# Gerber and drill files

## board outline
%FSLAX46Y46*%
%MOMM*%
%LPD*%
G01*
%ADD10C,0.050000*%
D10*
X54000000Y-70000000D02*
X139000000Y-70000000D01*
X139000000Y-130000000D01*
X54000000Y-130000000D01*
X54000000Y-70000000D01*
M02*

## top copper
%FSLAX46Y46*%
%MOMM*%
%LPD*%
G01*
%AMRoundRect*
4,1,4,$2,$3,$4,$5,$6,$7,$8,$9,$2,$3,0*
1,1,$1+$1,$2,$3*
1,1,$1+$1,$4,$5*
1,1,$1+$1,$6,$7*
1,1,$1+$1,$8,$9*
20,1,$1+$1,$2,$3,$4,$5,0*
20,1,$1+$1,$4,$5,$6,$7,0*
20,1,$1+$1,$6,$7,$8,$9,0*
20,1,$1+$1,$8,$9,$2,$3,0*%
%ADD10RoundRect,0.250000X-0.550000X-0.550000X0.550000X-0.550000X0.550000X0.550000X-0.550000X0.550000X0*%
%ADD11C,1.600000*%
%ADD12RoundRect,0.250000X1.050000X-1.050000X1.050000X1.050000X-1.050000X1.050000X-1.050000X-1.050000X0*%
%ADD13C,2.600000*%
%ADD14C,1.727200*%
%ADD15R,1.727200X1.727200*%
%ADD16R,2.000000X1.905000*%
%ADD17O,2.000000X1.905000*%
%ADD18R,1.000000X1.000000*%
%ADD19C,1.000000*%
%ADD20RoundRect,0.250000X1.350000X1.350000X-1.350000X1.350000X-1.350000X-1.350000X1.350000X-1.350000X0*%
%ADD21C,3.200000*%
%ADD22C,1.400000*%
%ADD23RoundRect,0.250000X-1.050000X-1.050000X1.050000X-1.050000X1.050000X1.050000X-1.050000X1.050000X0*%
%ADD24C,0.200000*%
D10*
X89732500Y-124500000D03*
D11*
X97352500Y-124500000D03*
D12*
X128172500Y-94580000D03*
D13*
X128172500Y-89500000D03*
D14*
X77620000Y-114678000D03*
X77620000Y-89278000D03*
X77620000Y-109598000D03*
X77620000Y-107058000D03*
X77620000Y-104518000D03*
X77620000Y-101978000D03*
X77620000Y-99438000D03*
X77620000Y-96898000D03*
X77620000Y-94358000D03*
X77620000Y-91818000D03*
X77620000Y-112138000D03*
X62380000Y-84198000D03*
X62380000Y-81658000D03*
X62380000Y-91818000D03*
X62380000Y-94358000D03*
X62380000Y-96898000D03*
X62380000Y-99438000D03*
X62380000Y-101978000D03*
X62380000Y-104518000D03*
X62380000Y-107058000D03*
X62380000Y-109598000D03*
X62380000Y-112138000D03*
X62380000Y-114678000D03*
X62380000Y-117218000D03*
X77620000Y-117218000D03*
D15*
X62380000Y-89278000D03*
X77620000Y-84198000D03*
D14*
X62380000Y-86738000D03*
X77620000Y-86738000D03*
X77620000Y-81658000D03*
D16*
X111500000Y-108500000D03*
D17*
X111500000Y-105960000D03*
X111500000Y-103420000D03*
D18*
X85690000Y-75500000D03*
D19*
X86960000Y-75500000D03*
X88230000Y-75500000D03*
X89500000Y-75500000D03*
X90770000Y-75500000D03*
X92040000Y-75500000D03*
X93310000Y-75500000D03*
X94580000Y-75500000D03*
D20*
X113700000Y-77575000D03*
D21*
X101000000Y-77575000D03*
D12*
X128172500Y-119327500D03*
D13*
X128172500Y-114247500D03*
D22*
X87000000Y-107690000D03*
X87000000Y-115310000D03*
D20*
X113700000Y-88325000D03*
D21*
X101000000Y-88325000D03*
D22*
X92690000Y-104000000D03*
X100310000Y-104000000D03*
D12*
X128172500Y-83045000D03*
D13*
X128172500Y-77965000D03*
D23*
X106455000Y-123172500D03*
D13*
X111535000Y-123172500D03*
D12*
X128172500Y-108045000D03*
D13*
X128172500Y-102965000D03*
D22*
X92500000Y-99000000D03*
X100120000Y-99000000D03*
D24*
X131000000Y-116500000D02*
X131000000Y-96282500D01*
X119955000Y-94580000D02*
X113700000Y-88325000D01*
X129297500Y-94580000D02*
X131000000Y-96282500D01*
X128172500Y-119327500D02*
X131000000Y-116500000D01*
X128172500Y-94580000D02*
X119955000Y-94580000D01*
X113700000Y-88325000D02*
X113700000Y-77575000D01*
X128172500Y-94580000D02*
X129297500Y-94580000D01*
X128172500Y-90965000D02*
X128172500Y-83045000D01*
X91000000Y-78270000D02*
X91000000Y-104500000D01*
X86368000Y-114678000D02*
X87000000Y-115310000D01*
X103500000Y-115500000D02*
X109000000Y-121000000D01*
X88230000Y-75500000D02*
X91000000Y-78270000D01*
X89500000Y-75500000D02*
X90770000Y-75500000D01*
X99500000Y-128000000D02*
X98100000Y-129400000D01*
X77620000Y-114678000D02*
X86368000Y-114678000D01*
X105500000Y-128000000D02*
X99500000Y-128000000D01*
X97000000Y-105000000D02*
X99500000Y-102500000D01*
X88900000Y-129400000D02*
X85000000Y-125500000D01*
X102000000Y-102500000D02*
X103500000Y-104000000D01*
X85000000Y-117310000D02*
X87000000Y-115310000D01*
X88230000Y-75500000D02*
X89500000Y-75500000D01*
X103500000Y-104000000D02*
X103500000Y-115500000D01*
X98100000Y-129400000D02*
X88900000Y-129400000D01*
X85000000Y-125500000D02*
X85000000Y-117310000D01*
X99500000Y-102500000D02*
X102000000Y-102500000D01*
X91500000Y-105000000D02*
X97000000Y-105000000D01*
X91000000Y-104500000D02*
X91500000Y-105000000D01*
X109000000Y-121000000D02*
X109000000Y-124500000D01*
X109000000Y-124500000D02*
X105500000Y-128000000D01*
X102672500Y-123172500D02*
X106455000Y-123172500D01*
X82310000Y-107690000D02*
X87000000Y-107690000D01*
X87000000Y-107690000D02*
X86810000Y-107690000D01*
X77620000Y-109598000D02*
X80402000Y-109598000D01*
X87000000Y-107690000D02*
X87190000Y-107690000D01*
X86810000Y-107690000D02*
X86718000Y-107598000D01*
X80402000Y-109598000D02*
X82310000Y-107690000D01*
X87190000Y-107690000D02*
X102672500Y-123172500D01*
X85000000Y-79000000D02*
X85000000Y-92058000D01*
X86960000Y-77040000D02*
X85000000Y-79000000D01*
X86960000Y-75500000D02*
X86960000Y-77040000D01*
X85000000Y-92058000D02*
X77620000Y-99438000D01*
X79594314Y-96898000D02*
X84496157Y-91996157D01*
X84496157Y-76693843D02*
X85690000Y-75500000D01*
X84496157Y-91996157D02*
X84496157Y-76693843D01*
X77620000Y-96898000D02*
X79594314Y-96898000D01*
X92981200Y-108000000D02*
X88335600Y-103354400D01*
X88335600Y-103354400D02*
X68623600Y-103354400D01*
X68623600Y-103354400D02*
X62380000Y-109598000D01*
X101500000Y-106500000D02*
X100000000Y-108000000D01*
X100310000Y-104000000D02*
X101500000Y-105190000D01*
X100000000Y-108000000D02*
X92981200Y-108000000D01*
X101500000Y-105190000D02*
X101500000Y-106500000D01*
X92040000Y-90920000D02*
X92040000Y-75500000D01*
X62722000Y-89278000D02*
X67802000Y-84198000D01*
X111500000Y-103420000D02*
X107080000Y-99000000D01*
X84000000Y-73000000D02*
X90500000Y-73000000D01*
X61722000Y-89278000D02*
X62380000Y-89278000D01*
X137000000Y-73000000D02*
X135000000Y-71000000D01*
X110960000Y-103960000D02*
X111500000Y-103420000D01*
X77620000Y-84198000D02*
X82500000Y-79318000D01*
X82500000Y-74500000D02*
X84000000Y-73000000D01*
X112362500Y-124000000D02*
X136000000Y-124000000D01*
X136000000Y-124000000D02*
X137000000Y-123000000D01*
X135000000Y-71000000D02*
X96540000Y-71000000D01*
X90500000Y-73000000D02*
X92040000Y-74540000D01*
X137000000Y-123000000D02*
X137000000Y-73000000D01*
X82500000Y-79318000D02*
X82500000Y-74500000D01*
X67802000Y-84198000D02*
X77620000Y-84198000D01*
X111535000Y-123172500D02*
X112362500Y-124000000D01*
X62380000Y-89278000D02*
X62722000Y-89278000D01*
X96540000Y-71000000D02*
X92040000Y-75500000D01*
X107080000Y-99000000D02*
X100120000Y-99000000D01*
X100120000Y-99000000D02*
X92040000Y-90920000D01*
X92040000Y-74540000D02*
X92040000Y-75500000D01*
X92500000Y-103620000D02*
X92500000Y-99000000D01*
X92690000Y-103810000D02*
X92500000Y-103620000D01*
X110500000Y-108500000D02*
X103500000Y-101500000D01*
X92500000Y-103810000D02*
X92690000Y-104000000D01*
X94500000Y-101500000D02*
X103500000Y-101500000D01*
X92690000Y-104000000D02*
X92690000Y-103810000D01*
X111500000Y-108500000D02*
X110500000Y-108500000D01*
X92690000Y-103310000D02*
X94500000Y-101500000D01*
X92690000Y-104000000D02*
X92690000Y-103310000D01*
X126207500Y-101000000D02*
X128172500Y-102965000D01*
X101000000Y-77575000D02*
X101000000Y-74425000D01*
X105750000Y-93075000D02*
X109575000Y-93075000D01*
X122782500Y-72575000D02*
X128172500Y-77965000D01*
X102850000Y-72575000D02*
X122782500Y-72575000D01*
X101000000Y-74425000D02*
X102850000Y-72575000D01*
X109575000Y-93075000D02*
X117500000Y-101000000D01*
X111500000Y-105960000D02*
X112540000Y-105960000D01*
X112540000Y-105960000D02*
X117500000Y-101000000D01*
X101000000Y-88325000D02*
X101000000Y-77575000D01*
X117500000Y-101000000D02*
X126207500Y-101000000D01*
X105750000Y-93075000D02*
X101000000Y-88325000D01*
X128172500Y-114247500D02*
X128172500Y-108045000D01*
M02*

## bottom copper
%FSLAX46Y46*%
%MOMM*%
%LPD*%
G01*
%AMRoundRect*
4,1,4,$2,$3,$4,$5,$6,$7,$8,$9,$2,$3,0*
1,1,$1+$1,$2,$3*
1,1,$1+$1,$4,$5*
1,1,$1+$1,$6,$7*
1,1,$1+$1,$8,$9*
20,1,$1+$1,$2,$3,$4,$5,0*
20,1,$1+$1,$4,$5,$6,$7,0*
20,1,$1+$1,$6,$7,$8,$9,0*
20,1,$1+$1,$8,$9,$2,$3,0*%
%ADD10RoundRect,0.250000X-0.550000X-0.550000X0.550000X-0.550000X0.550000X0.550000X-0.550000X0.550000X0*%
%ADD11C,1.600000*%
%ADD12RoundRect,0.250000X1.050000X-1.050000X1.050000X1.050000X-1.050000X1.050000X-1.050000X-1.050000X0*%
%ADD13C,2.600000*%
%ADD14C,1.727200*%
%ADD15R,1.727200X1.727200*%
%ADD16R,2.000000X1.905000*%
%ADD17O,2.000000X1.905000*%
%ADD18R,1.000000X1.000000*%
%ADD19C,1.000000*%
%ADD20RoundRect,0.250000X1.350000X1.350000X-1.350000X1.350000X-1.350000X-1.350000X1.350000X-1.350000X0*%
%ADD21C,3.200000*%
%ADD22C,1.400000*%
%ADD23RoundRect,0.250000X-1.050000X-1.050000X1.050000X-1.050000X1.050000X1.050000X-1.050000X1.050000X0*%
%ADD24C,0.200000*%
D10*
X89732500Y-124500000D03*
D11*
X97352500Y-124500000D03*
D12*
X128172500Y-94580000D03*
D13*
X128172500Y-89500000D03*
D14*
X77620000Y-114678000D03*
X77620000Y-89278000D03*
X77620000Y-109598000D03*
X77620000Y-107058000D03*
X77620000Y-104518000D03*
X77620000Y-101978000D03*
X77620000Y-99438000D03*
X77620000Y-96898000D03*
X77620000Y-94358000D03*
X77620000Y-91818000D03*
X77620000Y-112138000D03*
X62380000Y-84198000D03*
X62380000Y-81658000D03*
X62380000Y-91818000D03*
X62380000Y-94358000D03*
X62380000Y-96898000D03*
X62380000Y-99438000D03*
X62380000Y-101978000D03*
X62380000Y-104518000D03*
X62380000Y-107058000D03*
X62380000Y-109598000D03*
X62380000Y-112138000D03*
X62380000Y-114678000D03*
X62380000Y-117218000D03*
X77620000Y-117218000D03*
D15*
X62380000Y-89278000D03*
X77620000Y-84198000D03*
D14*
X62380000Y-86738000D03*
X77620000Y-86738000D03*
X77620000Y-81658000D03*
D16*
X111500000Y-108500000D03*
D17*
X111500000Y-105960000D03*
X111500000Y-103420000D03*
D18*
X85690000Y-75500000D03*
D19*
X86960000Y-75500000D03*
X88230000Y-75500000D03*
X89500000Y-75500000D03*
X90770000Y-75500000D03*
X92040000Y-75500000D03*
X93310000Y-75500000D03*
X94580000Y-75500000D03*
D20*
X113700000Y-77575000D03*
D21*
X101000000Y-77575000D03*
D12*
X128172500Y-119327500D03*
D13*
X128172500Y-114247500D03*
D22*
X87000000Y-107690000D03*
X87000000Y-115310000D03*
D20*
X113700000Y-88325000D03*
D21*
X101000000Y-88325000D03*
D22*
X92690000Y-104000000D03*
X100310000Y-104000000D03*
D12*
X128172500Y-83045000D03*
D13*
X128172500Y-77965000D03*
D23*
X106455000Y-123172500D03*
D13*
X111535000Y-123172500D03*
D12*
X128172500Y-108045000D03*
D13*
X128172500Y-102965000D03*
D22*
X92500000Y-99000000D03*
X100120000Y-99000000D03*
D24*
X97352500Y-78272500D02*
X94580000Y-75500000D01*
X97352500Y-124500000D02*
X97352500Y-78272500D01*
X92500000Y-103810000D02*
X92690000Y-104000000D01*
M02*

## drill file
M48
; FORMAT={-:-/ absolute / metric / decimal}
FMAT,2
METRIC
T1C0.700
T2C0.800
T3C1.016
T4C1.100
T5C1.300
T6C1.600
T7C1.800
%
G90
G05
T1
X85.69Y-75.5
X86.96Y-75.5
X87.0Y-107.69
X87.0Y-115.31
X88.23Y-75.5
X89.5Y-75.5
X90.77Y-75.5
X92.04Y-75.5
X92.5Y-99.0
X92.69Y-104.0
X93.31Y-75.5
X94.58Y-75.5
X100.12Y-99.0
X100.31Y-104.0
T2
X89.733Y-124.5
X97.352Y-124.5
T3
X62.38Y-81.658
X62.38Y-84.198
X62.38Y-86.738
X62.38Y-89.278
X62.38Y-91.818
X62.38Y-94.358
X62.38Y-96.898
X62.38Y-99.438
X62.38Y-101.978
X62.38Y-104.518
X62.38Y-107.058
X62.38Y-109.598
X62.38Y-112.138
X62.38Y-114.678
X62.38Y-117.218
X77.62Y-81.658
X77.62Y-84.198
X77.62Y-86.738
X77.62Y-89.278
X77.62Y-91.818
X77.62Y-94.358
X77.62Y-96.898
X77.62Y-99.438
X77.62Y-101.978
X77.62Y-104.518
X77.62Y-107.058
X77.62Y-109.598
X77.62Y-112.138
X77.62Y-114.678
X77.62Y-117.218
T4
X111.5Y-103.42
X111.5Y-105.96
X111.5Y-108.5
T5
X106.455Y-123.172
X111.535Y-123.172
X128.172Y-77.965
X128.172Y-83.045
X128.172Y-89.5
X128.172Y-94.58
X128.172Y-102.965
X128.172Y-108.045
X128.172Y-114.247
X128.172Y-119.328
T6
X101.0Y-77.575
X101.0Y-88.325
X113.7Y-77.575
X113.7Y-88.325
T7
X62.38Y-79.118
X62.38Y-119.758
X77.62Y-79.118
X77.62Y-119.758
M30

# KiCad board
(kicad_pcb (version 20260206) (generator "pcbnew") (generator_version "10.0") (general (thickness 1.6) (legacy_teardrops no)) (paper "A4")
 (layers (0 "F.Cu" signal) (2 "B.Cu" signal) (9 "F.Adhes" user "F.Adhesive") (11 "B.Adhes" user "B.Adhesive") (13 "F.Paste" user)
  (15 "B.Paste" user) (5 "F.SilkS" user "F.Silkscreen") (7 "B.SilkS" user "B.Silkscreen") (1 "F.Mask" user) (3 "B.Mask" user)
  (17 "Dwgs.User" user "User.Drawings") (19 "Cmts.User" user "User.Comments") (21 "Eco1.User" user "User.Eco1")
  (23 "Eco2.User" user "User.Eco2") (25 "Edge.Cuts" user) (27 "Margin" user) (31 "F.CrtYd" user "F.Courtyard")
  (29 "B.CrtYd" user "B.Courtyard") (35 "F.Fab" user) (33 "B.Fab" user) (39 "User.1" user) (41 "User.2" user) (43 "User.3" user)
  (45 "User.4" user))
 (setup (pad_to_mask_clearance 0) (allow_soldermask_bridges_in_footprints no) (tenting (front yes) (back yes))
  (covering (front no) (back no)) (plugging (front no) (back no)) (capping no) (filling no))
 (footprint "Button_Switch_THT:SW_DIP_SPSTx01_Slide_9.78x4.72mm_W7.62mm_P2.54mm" (layer "F.Cu") (at 89.7325 124.5)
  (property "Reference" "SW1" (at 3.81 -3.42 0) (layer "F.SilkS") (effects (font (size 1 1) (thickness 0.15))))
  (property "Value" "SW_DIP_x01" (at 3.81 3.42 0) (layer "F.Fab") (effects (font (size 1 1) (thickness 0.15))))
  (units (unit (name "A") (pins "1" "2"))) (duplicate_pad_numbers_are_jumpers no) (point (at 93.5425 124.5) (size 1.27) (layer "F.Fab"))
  (pad "1" thru_hole roundrect (at 0 0) (size 1.6 1.6) (drill 0.8) (layers "*.Cu" "*.Mask") (remove_unused_layers no)
   (roundrect_rratio 0.15625) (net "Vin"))
  (pad "2" thru_hole circle (at 7.62 0) (size 1.6 1.6) (drill 0.8) (layers "*.Cu" "*.Mask") (remove_unused_layers no) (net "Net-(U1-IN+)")))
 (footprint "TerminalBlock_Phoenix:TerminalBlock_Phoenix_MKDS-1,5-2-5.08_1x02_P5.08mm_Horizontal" (layer "F.Cu") (at 128.1725 94.58 90)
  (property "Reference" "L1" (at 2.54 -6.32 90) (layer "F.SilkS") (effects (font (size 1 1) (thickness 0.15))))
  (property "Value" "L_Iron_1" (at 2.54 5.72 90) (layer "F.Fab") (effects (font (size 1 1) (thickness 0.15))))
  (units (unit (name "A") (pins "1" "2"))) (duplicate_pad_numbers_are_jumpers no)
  (pad "1" thru_hole roundrect (at 0 0 90) (size 2.6 2.6) (drill 1.3) (layers "*.Cu" "*.Mask") (remove_unused_layers no)
   (roundrect_rratio 0.096154) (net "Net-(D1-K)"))
  (pad "2" thru_hole circle (at 5.08 0 90) (size 2.6 2.6) (drill 1.3) (layers "*.Cu" "*.Mask") (remove_unused_layers no)
   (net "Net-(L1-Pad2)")))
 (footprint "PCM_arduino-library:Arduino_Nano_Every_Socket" (layer "F.Cu") (at 70 121.028)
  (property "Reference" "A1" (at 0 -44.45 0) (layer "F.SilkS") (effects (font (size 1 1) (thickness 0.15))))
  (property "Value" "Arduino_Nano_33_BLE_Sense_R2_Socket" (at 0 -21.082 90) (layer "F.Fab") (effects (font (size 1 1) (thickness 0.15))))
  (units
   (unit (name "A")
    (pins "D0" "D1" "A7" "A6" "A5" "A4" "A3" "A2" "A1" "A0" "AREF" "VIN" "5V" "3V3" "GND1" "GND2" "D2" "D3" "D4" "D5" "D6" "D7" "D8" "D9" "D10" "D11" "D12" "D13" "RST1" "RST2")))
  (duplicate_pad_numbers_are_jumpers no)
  (pad "" np_thru_hole circle (at -7.62 -41.91) (size 1.8 1.8) (drill 1.8) (layers "*.Cu" "*.Mask"))
  (pad "" np_thru_hole circle (at -7.62 -1.27) (size 1.8 1.8) (drill 1.8) (layers "*.Cu" "*.Mask"))
  (pad "" np_thru_hole circle (at 7.62 -41.91) (size 1.8 1.8) (drill 1.8) (layers "*.Cu" "*.Mask"))
  (pad "" np_thru_hole circle (at 7.62 -1.27) (size 1.8 1.8) (drill 1.8) (layers "*.Cu" "*.Mask"))
  (pad "3V3" thru_hole circle (at 7.62 -6.35) (size 1.7272 1.7272) (drill 1.016) (layers "*.Cu" "*.Mask") (remove_unused_layers no)
   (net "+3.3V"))
  (pad "5V" thru_hole circle (at 7.62 -31.75) (size 1.7272 1.7272) (drill 1.016) (layers "*.Cu" "*.Mask") (remove_unused_layers no)
   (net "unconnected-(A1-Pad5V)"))
  (pad "A0" thru_hole circle (at 7.62 -11.43) (size 1.7272 1.7272) (drill 1.016) (layers "*.Cu" "*.Mask") (remove_unused_layers no)
   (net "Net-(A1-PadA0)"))
  (pad "A1" thru_hole circle (at 7.62 -13.97) (size 1.7272 1.7272) (drill 1.016) (layers "*.Cu" "*.Mask") (remove_unused_layers no)
   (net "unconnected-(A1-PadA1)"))
  (pad "A2" thru_hole circle (at 7.62 -16.51) (size 1.7272 1.7272) (drill 1.016) (layers "*.Cu" "*.Mask") (remove_unused_layers no)
   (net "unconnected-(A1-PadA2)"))
  (pad "A3" thru_hole circle (at 7.62 -19.05) (size 1.7272 1.7272) (drill 1.016) (layers "*.Cu" "*.Mask") (remove_unused_layers no)
   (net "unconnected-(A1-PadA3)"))
  (pad "A4" thru_hole circle (at 7.62 -21.59) (size 1.7272 1.7272) (drill 1.016) (layers "*.Cu" "*.Mask") (remove_unused_layers no)
   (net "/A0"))
  (pad "A5" thru_hole circle (at 7.62 -24.13) (size 1.7272 1.7272) (drill 1.016) (layers "*.Cu" "*.Mask") (remove_unused_layers no)
   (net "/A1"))
  (pad "A6" thru_hole circle (at 7.62 -26.67) (size 1.7272 1.7272) (drill 1.016) (layers "*.Cu" "*.Mask") (remove_unused_layers no)
   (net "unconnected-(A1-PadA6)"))
  (pad "A7" thru_hole circle (at 7.62 -29.21) (size 1.7272 1.7272) (drill 1.016) (layers "*.Cu" "*.Mask") (remove_unused_layers no)
   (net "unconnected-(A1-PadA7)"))
  (pad "AREF" thru_hole circle (at 7.62 -8.89) (size 1.7272 1.7272) (drill 1.016) (layers "*.Cu" "*.Mask") (remove_unused_layers no)
   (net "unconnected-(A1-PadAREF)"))
  (pad "D0" thru_hole circle (at -7.62 -36.83) (size 1.7272 1.7272) (drill 1.016) (layers "*.Cu" "*.Mask") (remove_unused_layers no)
   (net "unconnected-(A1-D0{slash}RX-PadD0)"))
  (pad "D1" thru_hole circle (at -7.62 -39.37) (size 1.7272 1.7272) (drill 1.016) (layers "*.Cu" "*.Mask") (remove_unused_layers no)
   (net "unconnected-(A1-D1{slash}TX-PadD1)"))
  (pad "D2" thru_hole circle (at -7.62 -29.21) (size 1.7272 1.7272) (drill 1.016) (layers "*.Cu" "*.Mask") (remove_unused_layers no)
   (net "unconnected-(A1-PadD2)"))
  (pad "D3" thru_hole circle (at -7.62 -26.67) (size 1.7272 1.7272) (drill 1.016) (layers "*.Cu" "*.Mask") (remove_unused_layers no)
   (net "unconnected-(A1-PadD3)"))
  (pad "D4" thru_hole circle (at -7.62 -24.13) (size 1.7272 1.7272) (drill 1.016) (layers "*.Cu" "*.Mask") (remove_unused_layers no)
   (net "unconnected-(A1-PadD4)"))
  (pad "D5" thru_hole circle (at -7.62 -21.59) (size 1.7272 1.7272) (drill 1.016) (layers "*.Cu" "*.Mask") (remove_unused_layers no)
   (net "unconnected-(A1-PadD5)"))
  (pad "D6" thru_hole circle (at -7.62 -19.05) (size 1.7272 1.7272) (drill 1.016) (layers "*.Cu" "*.Mask") (remove_unused_layers no)
   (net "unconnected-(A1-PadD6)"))
  (pad "D7" thru_hole circle (at -7.62 -16.51) (size 1.7272 1.7272) (drill 1.016) (layers "*.Cu" "*.Mask") (remove_unused_layers no)
   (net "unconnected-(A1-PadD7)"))
  (pad "D8" thru_hole circle (at -7.62 -13.97) (size 1.7272 1.7272) (drill 1.016) (layers "*.Cu" "*.Mask") (remove_unused_layers no)
   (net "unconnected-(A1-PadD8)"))
  (pad "D9" thru_hole circle (at -7.62 -11.43) (size 1.7272 1.7272) (drill 1.016) (layers "*.Cu" "*.Mask") (remove_unused_layers no)
   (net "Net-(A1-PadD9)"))
  (pad "D10" thru_hole circle (at -7.62 -8.89) (size 1.7272 1.7272) (drill 1.016) (layers "*.Cu" "*.Mask") (remove_unused_layers no)
   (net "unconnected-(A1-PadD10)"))
  (pad "D11" thru_hole circle (at -7.62 -6.35) (size 1.7272 1.7272) (drill 1.016) (layers "*.Cu" "*.Mask") (remove_unused_layers no)
   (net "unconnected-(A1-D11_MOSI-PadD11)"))
  (pad "D12" thru_hole circle (at -7.62 -3.81) (size 1.7272 1.7272) (drill 1.016) (layers "*.Cu" "*.Mask") (remove_unused_layers no)
   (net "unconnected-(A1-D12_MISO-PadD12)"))
  (pad "D13" thru_hole circle (at 7.62 -3.81) (size 1.7272 1.7272) (drill 1.016) (layers "*.Cu" "*.Mask") (remove_unused_layers no)
   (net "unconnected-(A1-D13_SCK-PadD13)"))
  (pad "GND1" thru_hole rect (at -7.62 -31.75) (size 1.7272 1.7272) (drill 1.016) (layers "*.Cu" "*.Mask") (remove_unused_layers no)
   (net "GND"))
  (pad "GND2" thru_hole rect (at 7.62 -36.83) (size 1.7272 1.7272) (drill 1.016) (layers "*.Cu" "*.Mask") (remove_unused_layers no)
   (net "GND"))
  (pad "RST1" thru_hole circle (at -7.62 -34.29) (size 1.7272 1.7272) (drill 1.016) (layers "*.Cu" "*.Mask") (remove_unused_layers no)
   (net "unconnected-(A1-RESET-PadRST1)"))
  (pad "RST2" thru_hole circle (at 7.62 -34.29) (size 1.7272 1.7272) (drill 1.016) (layers "*.Cu" "*.Mask") (remove_unused_layers no)
   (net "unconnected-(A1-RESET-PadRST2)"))
  (pad "VIN" thru_hole circle (at 7.62 -39.37) (size 1.7272 1.7272) (drill 1.016) (layers "*.Cu" "*.Mask") (remove_unused_layers no)
   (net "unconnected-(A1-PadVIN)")))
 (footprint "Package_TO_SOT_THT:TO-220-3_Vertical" (layer "F.Cu") (at 111.5 108.5 90)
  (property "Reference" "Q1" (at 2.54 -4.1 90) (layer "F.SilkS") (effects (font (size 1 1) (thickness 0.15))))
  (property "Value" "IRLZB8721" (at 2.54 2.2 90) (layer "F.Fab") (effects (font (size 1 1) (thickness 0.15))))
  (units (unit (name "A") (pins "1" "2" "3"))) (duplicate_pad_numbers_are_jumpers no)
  (pad "1" thru_hole rect (at 0 0 90) (size 1.905 2) (drill 1.1) (layers "*.Cu" "*.Mask") (remove_unused_layers no) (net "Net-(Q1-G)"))
  (pad "2" thru_hole oval (at 2.54 0 90) (size 1.905 2) (drill 1.1) (layers "*.Cu" "*.Mask") (remove_unused_layers no) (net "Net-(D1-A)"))
  (pad "3" thru_hole oval (at 5.08 0 90) (size 1.905 2) (drill 1.1) (layers "*.Cu" "*.Mask") (remove_unused_layers no) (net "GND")))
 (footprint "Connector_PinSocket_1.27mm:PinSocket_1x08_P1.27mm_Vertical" (layer "F.Cu") (at 85.69 75.5 90)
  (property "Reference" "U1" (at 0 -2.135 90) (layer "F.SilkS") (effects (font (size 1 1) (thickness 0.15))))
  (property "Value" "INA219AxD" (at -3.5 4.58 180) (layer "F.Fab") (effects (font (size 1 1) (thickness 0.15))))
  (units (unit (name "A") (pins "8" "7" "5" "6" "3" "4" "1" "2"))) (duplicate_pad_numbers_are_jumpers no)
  (pad "1" thru_hole rect (at 0 0 90) (size 1 1) (drill 0.7) (layers "*.Cu" "*.Mask") (remove_unused_layers no) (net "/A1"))
  (pad "2" thru_hole circle (at 0 1.27 90) (size 1 1) (drill 0.7) (layers "*.Cu" "*.Mask") (remove_unused_layers no) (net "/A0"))
  (pad "3" thru_hole circle (at 0 2.54 90) (size 1 1) (drill 0.7) (layers "*.Cu" "*.Mask") (remove_unused_layers no) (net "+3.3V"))
  (pad "4" thru_hole circle (at 0 3.81 90) (size 1 1) (drill 0.7) (layers "*.Cu" "*.Mask") (remove_unused_layers no) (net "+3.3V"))
  (pad "5" thru_hole circle (at 0 5.08 90) (size 1 1) (drill 0.7) (layers "*.Cu" "*.Mask") (remove_unused_layers no) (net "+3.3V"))
  (pad "6" thru_hole circle (at 0 6.35 90) (size 1 1) (drill 0.7) (layers "*.Cu" "*.Mask") (remove_unused_layers no) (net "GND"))
  (pad "7" thru_hole circle (at 0 7.62 90) (size 1 1) (drill 0.7) (layers "*.Cu" "*.Mask") (remove_unused_layers no) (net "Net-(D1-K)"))
  (pad "8" thru_hole circle (at 0 8.89 90) (size 1 1) (drill 0.7) (layers "*.Cu" "*.Mask") (remove_unused_layers no) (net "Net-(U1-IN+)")))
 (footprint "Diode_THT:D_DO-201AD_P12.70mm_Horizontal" (layer "F.Cu") (at 113.7 77.575 180)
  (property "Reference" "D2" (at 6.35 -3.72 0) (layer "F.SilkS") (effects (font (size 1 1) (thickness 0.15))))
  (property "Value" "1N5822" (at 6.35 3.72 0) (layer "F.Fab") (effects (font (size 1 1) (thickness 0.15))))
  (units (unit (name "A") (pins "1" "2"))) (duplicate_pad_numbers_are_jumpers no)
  (pad "1" thru_hole roundrect (at 0 0 180) (size 3.2 3.2) (drill 1.6) (layers "*.Cu" "*.Mask") (remove_unused_layers no)
   (roundrect_rratio 0.078125) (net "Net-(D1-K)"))
  (pad "2" thru_hole circle (at 12.7 0 180) (size 3.2 3.2) (drill 1.6) (layers "*.Cu" "*.Mask") (remove_unused_layers no) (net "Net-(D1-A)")))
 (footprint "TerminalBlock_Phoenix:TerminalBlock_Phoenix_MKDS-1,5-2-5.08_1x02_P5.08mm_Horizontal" (layer "F.Cu") (at 128.1725 119.3275 90)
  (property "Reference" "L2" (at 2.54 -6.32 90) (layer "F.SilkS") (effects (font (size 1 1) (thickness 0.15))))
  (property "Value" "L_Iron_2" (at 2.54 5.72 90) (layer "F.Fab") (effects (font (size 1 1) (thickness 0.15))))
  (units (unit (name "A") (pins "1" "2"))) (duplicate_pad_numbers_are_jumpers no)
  (pad "1" thru_hole roundrect (at 0 0 90) (size 2.6 2.6) (drill 1.3) (layers "*.Cu" "*.Mask") (remove_unused_layers no)
   (roundrect_rratio 0.096154) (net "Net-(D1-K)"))
  (pad "2" thru_hole circle (at 5.08 0 90) (size 2.6 2.6) (drill 1.3) (layers "*.Cu" "*.Mask") (remove_unused_layers no)
   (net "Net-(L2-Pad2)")))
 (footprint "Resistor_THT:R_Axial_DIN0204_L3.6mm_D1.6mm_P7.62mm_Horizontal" (layer "F.Cu") (at 87 107.69 -90)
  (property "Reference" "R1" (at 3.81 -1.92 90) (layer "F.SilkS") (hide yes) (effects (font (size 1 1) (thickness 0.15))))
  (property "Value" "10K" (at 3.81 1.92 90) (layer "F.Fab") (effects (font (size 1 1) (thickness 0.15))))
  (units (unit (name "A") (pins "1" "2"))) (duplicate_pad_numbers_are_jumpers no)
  (pad "1" thru_hole circle (at 0 0 270) (size 1.4 1.4) (drill 0.7) (layers "*.Cu" "*.Mask") (remove_unused_layers no)
   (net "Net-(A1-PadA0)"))
  (pad "2" thru_hole circle (at 7.62 0 270) (size 1.4 1.4) (drill 0.7) (layers "*.Cu" "*.Mask") (remove_unused_layers no) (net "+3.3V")))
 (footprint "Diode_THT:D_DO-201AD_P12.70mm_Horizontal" (layer "F.Cu") (at 113.7 88.325 180)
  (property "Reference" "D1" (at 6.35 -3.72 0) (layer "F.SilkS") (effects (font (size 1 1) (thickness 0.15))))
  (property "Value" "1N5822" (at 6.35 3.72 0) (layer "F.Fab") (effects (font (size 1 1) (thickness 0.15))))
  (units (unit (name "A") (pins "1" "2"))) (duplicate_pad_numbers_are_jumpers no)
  (pad "1" thru_hole roundrect (at 0 0 180) (size 3.2 3.2) (drill 1.6) (layers "*.Cu" "*.Mask") (remove_unused_layers no)
   (roundrect_rratio 0.078125) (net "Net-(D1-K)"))
  (pad "2" thru_hole circle (at 12.7 0 180) (size 3.2 3.2) (drill 1.6) (layers "*.Cu" "*.Mask") (remove_unused_layers no) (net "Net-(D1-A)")))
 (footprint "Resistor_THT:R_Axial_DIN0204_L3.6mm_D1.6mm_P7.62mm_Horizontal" (layer "F.Cu") (at 92.69 104)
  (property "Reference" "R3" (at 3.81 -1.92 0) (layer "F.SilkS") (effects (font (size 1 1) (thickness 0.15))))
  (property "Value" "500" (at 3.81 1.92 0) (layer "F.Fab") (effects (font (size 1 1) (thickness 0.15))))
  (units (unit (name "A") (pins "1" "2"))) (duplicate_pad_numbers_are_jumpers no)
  (pad "1" thru_hole circle (at 0 0) (size 1.4 1.4) (drill 0.7) (layers "*.Cu" "*.Mask") (remove_unused_layers no) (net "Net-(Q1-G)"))
  (pad "2" thru_hole circle (at 7.62 0) (size 1.4 1.4) (drill 0.7) (layers "*.Cu" "*.Mask") (remove_unused_layers no) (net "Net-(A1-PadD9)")))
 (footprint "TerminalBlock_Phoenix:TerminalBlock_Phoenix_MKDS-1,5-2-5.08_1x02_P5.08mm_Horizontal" (layer "F.Cu") (at 128.1725 83.045 90)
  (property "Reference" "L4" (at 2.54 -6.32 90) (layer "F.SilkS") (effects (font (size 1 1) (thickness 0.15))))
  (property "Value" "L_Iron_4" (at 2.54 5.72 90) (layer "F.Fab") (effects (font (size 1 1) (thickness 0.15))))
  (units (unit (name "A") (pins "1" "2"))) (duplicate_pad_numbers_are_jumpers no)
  (pad "1" thru_hole roundrect (at 0 0 90) (size 2.6 2.6) (drill 1.3) (layers "*.Cu" "*.Mask") (remove_unused_layers no)
   (roundrect_rratio 0.096154) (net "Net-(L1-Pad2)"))
  (pad "2" thru_hole circle (at 5.08 0 90) (size 2.6 2.6) (drill 1.3) (layers "*.Cu" "*.Mask") (remove_unused_layers no) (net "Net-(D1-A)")))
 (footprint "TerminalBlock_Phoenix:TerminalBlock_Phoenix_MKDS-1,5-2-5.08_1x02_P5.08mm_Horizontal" (layer "F.Cu") (at 106.455 123.1725)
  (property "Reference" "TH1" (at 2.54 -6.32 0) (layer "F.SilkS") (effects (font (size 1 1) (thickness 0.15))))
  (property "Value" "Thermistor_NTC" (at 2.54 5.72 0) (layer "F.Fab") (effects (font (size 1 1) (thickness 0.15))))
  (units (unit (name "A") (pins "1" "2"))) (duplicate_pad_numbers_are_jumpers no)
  (pad "1" thru_hole roundrect (at 0 0) (size 2.6 2.6) (drill 1.3) (layers "*.Cu" "*.Mask") (remove_unused_layers no)
   (roundrect_rratio 0.096154) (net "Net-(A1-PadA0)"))
  (pad "2" thru_hole circle (at 5.08 0) (size 2.6 2.6) (drill 1.3) (layers "*.Cu" "*.Mask") (remove_unused_layers no) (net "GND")))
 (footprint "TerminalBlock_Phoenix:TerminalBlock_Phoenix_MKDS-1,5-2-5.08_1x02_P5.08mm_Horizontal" (layer "F.Cu") (at 128.1725 108.045 90)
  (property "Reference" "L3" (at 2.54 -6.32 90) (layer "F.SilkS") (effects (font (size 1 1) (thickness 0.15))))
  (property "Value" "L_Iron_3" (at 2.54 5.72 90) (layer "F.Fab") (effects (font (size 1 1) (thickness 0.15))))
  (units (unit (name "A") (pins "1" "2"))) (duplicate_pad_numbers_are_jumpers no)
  (pad "1" thru_hole roundrect (at 0 0 90) (size 2.6 2.6) (drill 1.3) (layers "*.Cu" "*.Mask") (remove_unused_layers no)
   (roundrect_rratio 0.096154) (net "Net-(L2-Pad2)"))
  (pad "2" thru_hole circle (at 5.08 0 90) (size 2.6 2.6) (drill 1.3) (layers "*.Cu" "*.Mask") (remove_unused_layers no) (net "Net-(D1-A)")))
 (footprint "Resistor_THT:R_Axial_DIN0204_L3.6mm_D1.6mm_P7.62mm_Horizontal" (layer "F.Cu") (at 92.5 99)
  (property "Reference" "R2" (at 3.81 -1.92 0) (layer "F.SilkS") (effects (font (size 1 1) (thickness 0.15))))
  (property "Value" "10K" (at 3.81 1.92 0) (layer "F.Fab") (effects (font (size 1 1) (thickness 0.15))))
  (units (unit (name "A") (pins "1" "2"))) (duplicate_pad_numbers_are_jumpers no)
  (pad "1" thru_hole circle (at 0 0) (size 1.4 1.4) (drill 0.7) (layers "*.Cu" "*.Mask") (remove_unused_layers no) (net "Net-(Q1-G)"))
  (pad "2" thru_hole circle (at 7.62 0) (size 1.4 1.4) (drill 0.7) (layers "*.Cu" "*.Mask") (remove_unused_layers no) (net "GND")))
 (gr_rect (start 54 70) (end 139 130) (stroke (width 0.05) (type default)) (fill no) (layer "Edge.Cuts"))
 (segment (start 97.3525 78.2725) (end 94.58 75.5) (width 0.2) (layer "B.Cu") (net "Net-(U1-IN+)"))
 (segment (start 97.3525 124.5) (end 97.3525 78.2725) (width 0.2) (layer "B.Cu") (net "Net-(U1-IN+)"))
 (segment (start 131 116.5) (end 131 96.2825) (width 0.2) (layer "F.Cu") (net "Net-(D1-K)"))
 (segment (start 119.955 94.58) (end 113.7 88.325) (width 0.2) (layer "F.Cu") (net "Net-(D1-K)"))
 (segment (start 129.2975 94.58) (end 131 96.2825) (width 0.2) (layer "F.Cu") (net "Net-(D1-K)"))
 (segment (start 128.1725 119.3275) (end 131 116.5) (width 0.2) (layer "F.Cu") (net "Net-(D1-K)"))
 (segment (start 128.1725 94.58) (end 119.955 94.58) (width 0.2) (layer "F.Cu") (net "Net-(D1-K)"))
 (segment (start 113.7 88.325) (end 113.7 77.575) (width 0.2) (layer "F.Cu") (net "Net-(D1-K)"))
 (segment (start 128.1725 94.58) (end 129.2975 94.58) (width 0.2) (layer "F.Cu") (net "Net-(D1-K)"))
 (segment (start 128.1725 90.965) (end 128.1725 83.045) (width 0.2) (layer "F.Cu") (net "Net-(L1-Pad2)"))
 (segment (start 91 78.27) (end 91 104.5) (width 0.2) (layer "F.Cu") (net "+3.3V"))
 (segment (start 86.368 114.678) (end 87 115.31) (width 0.2) (layer "F.Cu") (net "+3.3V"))
 (segment (start 103.5 115.5) (end 109 121) (width 0.2) (layer "F.Cu") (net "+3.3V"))
 (segment (start 88.23 75.5) (end 91 78.27) (width 0.2) (layer "F.Cu") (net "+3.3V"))
 (segment (start 89.5 75.5) (end 90.77 75.5) (width 0.2) (layer "F.Cu") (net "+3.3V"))
 (segment (start 99.5 128) (end 98.1 129.4) (width 0.2) (layer "F.Cu") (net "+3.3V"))
 (segment (start 77.62 114.678) (end 86.368 114.678) (width 0.2) (layer "F.Cu") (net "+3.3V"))
 (segment (start 105.5 128) (end 99.5 128) (width 0.2) (layer "F.Cu") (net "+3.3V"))
 (segment (start 97 105) (end 99.5 102.5) (width 0.2) (layer "F.Cu") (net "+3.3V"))
 (segment (start 88.9 129.4) (end 85 125.5) (width 0.2) (layer "F.Cu") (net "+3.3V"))
 (segment (start 102 102.5) (end 103.5 104) (width 0.2) (layer "F.Cu") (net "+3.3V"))
 (segment (start 85 117.31) (end 87 115.31) (width 0.2) (layer "F.Cu") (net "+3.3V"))
 (segment (start 88.23 75.5) (end 89.5 75.5) (width 0.2) (layer "F.Cu") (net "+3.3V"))
 (segment (start 103.5 104) (end 103.5 115.5) (width 0.2) (layer "F.Cu") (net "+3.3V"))
 (segment (start 98.1 129.4) (end 88.9 129.4) (width 0.2) (layer "F.Cu") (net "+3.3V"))
 (segment (start 85 125.5) (end 85 117.31) (width 0.2) (layer "F.Cu") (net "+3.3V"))
 (segment (start 99.5 102.5) (end 102 102.5) (width 0.2) (layer "F.Cu") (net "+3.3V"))
 (segment (start 91.5 105) (end 97 105) (width 0.2) (layer "F.Cu") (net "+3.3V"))
 (segment (start 91 104.5) (end 91.5 105) (width 0.2) (layer "F.Cu") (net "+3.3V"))
 (segment (start 109 121) (end 109 124.5) (width 0.2) (layer "F.Cu") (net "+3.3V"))
 (segment (start 109 124.5) (end 105.5 128) (width 0.2) (layer "F.Cu") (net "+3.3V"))
 (segment (start 102.6725 123.1725) (end 106.455 123.1725) (width 0.2) (layer "F.Cu") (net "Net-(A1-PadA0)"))
 (segment (start 82.31 107.69) (end 87 107.69) (width 0.2) (layer "F.Cu") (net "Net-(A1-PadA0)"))
 (segment (start 87 107.69) (end 86.81 107.69) (width 0.2) (layer "F.Cu") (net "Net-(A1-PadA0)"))
 (segment (start 77.62 109.598) (end 80.402 109.598) (width 0.2) (layer "F.Cu") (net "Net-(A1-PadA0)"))
 (segment (start 87 107.69) (end 87.19 107.69) (width 0.2) (layer "F.Cu") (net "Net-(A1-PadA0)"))
 (segment (start 86.81 107.69) (end 86.718 107.598) (width 0.2) (layer "F.Cu") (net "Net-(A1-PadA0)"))
 (segment (start 80.402 109.598) (end 82.31 107.69) (width 0.2) (layer "F.Cu") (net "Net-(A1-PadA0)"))
 (segment (start 87.19 107.69) (end 102.6725 123.1725) (width 0.2) (layer "F.Cu") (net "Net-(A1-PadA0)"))
 (segment (start 85 79) (end 85 92.058) (width 0.2) (layer "F.Cu") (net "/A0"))
 (segment (start 86.96 77.04) (end 85 79) (width 0.2) (layer "F.Cu") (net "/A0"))
 (segment (start 86.96 75.5) (end 86.96 77.04) (width 0.2) (layer "F.Cu") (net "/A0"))
 (segment (start 85 92.058) (end 77.62 99.438) (width 0.2) (layer "F.Cu") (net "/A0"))
 (segment (start 79.594314 96.898) (end 84.496157 91.996157) (width 0.2) (layer "F.Cu") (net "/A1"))
 (segment (start 84.496157 76.693843) (end 85.69 75.5) (width 0.2) (layer "F.Cu") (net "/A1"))
 (segment (start 84.496157 91.996157) (end 84.496157 76.693843) (width 0.2) (layer "F.Cu") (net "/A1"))
 (segment (start 77.62 96.898) (end 79.594314 96.898) (width 0.2) (layer "F.Cu") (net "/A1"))
 (segment (start 92.9812 108) (end 88.3356 103.3544) (width 0.2) (layer "F.Cu") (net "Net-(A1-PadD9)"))
 (segment (start 88.3356 103.3544) (end 68.6236 103.3544) (width 0.2) (layer "F.Cu") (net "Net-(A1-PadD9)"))
 (segment (start 68.6236 103.3544) (end 62.38 109.598) (width 0.2) (layer "F.Cu") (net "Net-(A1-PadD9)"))
 (segment (start 101.5 106.5) (end 100 108) (width 0.2) (layer "F.Cu") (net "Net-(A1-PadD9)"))
 (segment (start 100.31 104) (end 101.5 105.19) (width 0.2) (layer "F.Cu") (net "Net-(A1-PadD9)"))
 (segment (start 100 108) (end 92.9812 108) (width 0.2) (layer "F.Cu") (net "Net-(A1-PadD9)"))
 (segment (start 101.5 105.19) (end 101.5 106.5) (width 0.2) (layer "F.Cu") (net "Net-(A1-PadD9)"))
 (segment (start 92.04 90.92) (end 92.04 75.5) (width 0.2) (layer "F.Cu") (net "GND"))
 (segment (start 62.722 89.278) (end 67.802 84.198) (width 0.2) (layer "F.Cu") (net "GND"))
 (segment (start 111.5 103.42) (end 107.08 99) (width 0.2) (layer "F.Cu") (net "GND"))
 (segment (start 84 73) (end 90.5 73) (width 0.2) (layer "F.Cu") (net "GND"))
 (segment (start 61.722 89.278) (end 62.38 89.278) (width 0.2) (layer "F.Cu") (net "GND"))
 (segment (start 137 73) (end 135 71) (width 0.2) (layer "F.Cu") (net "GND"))
 (segment (start 110.96 103.96) (end 111.5 103.42) (width 0.2) (layer "F.Cu") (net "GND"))
 (segment (start 77.62 84.198) (end 82.5 79.318) (width 0.2) (layer "F.Cu") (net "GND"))
 (segment (start 82.5 74.5) (end 84 73) (width 0.2) (layer "F.Cu") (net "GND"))
 (segment (start 112.3625 124) (end 136 124) (width 0.2) (layer "F.Cu") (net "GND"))
 (segment (start 136 124) (end 137 123) (width 0.2) (layer "F.Cu") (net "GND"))
 (segment (start 135 71) (end 96.54 71) (width 0.2) (layer "F.Cu") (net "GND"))
 (segment (start 90.5 73) (end 92.04 74.54) (width 0.2) (layer "F.Cu") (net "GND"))
 (segment (start 137 123) (end 137 73) (width 0.2) (layer "F.Cu") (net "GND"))
 (segment (start 82.5 79.318) (end 82.5 74.5) (width 0.2) (layer "F.Cu") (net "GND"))
 (segment (start 67.802 84.198) (end 77.62 84.198) (width 0.2) (layer "F.Cu") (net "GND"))
 (segment (start 111.535 123.1725) (end 112.3625 124) (width 0.2) (layer "F.Cu") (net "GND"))
 (segment (start 62.38 89.278) (end 62.722 89.278) (width 0.2) (layer "F.Cu") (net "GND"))
 (segment (start 96.54 71) (end 92.04 75.5) (width 0.2) (layer "F.Cu") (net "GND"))
 (segment (start 107.08 99) (end 100.12 99) (width 0.2) (layer "F.Cu") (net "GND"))
 (segment (start 100.12 99) (end 92.04 90.92) (width 0.2) (layer "F.Cu") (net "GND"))
 (segment (start 92.04 74.54) (end 92.04 75.5) (width 0.2) (layer "F.Cu") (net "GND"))
 (segment (start 92.5 103.62) (end 92.5 99) (width 0.2) (layer "F.Cu") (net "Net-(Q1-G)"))
 (segment (start 92.69 103.81) (end 92.5 103.62) (width 0.2) (layer "F.Cu") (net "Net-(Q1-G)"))
 (segment (start 110.5 108.5) (end 103.5 101.5) (width 0.2) (layer "F.Cu") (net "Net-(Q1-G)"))
 (segment (start 92.5 103.81) (end 92.69 104) (width 0.2) (layer "F.Cu") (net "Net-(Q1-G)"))
 (segment (start 94.5 101.5) (end 103.5 101.5) (width 0.2) (layer "F.Cu") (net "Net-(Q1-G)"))
 (segment (start 92.69 104) (end 92.69 103.81) (width 0.2) (layer "F.Cu") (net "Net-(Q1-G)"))
 (segment (start 111.5 108.5) (end 110.5 108.5) (width 0.2) (layer "F.Cu") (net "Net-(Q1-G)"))
 (segment (start 92.69 103.31) (end 94.5 101.5) (width 0.2) (layer "F.Cu") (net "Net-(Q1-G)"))
 (segment (start 92.69 104) (end 92.69 103.31) (width 0.2) (layer "F.Cu") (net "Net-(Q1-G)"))
 (segment (start 92.5 103.81) (end 92.69 104) (width 0.2) (layer "B.Cu") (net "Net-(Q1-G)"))
 (segment (start 126.2075 101) (end 128.1725 102.965) (width 0.2) (layer "F.Cu") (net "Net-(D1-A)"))
 (segment (start 101 77.575) (end 101 74.425) (width 0.2) (layer "F.Cu") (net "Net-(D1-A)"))
 (segment (start 105.75 93.075) (end 109.575 93.075) (width 0.2) (layer "F.Cu") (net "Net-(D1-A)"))
 (segment (start 122.7825 72.575) (end 128.1725 77.965) (width 0.2) (layer "F.Cu") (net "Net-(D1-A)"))
 (segment (start 102.85 72.575) (end 122.7825 72.575) (width 0.2) (layer "F.Cu") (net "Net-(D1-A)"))
 (segment (start 101 74.425) (end 102.85 72.575) (width 0.2) (layer "F.Cu") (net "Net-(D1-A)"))
 (segment (start 109.575 93.075) (end 117.5 101) (width 0.2) (layer "F.Cu") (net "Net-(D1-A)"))
 (segment (start 111.5 105.96) (end 112.54 105.96) (width 0.2) (layer "F.Cu") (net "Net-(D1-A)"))
 (segment (start 112.54 105.96) (end 117.5 101) (width 0.2) (layer "F.Cu") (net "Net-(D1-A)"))
 (segment (start 101 88.325) (end 101 77.575) (width 0.2) (layer "F.Cu") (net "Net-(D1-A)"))
 (segment (start 117.5 101) (end 126.2075 101) (width 0.2) (layer "F.Cu") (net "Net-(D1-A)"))
 (segment (start 105.75 93.075) (end 101 88.325) (width 0.2) (layer "F.Cu") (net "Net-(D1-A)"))
 (segment (start 128.1725 114.2475) (end 128.1725 108.045) (width 0.2) (layer "F.Cu") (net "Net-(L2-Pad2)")))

